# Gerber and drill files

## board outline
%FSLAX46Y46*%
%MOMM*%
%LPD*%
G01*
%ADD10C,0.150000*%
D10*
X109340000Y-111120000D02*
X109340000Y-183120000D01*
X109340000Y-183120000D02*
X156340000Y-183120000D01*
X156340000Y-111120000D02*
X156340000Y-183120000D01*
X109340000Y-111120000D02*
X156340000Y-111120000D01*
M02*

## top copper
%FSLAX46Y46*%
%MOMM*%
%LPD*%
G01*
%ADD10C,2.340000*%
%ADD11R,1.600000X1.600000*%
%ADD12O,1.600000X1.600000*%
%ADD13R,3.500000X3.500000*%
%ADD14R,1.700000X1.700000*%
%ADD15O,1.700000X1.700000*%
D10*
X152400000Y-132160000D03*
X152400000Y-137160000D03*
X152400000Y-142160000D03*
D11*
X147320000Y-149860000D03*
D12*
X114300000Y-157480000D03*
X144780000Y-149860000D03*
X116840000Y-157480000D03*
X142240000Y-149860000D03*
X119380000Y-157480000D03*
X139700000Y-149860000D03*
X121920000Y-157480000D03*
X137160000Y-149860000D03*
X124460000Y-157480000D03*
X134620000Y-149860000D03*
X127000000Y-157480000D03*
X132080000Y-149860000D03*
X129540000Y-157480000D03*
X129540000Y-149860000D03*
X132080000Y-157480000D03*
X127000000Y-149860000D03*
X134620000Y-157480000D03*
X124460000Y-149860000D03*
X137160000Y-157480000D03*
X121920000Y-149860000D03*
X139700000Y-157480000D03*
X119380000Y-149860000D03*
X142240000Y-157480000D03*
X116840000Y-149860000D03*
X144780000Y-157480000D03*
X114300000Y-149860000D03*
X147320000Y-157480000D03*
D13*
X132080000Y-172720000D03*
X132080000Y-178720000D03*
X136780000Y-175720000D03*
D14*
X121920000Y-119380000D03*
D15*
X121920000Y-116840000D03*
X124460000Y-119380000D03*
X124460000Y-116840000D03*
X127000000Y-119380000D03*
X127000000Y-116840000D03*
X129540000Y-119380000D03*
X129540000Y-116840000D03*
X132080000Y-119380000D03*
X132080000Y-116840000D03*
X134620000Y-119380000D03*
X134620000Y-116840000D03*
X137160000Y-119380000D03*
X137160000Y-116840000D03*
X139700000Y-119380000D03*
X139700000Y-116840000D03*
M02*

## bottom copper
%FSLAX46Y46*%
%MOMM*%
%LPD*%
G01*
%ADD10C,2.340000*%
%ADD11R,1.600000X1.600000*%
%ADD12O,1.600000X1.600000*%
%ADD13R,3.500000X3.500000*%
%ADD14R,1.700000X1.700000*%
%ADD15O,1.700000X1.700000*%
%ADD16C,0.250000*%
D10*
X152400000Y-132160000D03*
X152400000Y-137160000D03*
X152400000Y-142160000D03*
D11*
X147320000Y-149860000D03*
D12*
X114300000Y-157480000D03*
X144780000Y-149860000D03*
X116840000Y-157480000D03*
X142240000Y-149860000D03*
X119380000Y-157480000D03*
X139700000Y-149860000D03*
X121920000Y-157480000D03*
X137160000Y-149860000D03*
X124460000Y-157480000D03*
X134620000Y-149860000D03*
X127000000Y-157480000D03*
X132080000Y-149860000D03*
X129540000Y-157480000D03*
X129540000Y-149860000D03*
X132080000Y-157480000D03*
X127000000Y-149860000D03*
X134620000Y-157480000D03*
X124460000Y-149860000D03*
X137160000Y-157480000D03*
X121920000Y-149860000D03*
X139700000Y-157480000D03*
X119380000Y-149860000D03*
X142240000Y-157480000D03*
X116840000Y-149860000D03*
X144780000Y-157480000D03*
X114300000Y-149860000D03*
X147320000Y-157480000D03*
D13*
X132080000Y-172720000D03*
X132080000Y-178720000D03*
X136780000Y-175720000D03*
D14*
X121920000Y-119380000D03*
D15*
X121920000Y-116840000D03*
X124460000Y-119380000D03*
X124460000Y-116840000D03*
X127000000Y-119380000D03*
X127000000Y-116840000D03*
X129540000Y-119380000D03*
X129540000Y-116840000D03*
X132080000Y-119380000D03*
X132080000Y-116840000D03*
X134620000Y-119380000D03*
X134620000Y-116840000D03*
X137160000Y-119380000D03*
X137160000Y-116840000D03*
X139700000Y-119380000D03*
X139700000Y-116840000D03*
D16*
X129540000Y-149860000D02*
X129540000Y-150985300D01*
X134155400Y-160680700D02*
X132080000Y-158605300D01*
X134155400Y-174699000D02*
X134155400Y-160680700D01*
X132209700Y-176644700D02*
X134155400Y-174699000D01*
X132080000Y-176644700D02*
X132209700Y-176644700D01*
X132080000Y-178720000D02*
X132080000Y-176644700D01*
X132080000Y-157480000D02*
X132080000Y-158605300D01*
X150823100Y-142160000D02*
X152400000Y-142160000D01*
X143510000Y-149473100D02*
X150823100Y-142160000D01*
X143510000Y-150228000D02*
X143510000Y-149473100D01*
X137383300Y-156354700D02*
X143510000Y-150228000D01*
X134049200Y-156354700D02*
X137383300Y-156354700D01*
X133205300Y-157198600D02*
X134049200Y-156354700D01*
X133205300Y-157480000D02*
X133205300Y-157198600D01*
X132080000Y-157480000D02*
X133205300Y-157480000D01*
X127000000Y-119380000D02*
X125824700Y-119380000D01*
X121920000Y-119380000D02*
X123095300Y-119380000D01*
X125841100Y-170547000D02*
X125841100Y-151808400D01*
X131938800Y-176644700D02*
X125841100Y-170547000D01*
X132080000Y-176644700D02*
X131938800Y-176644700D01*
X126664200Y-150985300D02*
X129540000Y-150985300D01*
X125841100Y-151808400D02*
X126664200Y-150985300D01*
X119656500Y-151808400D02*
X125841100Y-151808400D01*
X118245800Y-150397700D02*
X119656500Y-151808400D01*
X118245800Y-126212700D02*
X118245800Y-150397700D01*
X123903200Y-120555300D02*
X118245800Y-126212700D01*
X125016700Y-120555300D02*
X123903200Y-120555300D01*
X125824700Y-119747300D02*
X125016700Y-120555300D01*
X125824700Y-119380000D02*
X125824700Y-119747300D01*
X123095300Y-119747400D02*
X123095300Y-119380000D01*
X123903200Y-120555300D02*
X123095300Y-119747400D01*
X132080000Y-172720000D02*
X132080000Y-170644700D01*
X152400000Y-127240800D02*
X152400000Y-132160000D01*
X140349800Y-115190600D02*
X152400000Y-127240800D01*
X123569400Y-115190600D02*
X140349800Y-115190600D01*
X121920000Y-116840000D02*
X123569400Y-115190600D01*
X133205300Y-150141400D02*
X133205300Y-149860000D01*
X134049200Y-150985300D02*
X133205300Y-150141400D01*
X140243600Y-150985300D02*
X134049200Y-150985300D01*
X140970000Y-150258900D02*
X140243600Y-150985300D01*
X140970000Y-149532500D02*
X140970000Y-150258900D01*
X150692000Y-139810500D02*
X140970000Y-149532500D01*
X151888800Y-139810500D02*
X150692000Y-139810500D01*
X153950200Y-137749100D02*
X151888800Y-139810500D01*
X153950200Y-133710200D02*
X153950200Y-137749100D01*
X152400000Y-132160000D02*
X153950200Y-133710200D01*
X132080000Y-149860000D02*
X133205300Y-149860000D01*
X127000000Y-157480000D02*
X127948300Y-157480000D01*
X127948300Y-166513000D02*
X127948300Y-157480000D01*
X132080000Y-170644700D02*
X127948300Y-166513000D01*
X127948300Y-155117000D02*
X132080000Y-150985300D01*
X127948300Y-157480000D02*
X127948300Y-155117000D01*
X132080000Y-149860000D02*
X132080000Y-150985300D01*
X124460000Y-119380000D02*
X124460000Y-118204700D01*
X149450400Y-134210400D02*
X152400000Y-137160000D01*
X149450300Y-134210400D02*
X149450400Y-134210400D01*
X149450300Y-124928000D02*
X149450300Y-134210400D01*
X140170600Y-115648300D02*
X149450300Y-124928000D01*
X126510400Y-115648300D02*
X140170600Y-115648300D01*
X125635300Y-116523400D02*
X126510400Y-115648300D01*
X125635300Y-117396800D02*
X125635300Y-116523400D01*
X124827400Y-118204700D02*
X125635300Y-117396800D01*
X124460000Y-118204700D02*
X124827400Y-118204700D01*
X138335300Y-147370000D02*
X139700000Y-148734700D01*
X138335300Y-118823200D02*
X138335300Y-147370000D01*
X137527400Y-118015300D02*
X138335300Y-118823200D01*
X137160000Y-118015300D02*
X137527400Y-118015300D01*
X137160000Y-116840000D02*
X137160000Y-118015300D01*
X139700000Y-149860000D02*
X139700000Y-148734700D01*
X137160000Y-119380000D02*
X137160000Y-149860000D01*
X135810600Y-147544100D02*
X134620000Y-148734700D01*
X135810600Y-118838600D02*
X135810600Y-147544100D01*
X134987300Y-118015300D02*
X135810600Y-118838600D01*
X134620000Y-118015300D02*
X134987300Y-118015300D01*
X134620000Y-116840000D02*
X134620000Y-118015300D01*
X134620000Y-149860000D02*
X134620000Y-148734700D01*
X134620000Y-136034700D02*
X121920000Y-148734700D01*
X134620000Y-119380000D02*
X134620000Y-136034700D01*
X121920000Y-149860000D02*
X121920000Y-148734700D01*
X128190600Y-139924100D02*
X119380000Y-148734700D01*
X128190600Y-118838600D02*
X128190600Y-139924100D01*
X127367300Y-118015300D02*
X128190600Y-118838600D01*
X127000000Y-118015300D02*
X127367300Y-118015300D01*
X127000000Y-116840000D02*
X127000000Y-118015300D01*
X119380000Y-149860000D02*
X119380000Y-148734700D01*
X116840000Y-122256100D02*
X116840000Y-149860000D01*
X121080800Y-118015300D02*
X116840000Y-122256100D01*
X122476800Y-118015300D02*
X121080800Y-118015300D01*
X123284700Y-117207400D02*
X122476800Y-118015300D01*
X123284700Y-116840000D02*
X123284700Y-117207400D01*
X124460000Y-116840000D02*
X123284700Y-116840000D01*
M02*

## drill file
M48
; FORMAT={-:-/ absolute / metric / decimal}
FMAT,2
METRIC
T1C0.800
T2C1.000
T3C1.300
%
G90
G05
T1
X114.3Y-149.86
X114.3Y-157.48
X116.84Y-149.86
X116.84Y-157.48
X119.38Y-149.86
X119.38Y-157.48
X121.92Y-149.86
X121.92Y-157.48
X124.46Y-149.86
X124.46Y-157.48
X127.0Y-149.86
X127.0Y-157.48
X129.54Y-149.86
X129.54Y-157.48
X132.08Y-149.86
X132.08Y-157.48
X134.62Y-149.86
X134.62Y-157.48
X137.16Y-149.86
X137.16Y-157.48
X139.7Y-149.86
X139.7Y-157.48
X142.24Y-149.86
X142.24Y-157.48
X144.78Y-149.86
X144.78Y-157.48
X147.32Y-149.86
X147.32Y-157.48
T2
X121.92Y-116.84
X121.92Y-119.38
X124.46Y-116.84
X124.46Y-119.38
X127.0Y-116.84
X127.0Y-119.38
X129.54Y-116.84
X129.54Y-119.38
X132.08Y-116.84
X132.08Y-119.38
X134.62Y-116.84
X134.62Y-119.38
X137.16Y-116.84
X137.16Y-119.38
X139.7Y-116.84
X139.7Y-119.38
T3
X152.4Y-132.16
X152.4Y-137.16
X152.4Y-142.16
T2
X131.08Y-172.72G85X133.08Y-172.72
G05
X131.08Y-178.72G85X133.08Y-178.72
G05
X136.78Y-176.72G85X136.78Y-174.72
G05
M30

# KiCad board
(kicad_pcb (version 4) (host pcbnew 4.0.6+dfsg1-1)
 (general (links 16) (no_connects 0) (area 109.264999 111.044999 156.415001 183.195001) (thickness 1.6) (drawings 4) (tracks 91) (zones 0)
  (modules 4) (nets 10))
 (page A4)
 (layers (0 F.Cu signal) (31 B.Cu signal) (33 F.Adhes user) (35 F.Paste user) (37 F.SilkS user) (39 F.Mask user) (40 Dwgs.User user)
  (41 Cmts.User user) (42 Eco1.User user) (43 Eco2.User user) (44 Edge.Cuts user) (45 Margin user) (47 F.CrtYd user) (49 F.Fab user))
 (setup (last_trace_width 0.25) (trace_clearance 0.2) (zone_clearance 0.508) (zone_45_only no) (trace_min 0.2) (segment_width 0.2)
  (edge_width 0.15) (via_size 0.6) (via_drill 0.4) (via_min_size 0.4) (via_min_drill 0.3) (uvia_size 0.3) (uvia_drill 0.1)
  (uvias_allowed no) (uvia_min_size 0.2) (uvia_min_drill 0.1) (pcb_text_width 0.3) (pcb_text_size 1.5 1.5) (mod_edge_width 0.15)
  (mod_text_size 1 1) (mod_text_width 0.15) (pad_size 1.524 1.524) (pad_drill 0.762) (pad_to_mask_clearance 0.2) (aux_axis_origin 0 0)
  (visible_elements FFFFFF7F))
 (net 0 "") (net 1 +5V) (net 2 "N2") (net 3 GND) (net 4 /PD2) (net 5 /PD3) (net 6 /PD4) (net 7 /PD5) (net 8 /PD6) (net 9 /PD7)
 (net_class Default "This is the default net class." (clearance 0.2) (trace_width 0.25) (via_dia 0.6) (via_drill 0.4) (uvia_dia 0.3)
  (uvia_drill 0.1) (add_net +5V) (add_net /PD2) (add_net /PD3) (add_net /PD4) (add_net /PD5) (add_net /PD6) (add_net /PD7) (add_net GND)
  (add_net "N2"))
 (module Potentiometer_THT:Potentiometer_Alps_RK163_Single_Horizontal (layer F.Cu) (at 152.4 142.16)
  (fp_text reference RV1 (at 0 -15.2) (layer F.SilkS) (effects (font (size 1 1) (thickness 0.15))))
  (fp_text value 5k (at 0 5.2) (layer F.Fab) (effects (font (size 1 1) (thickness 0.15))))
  (pad 3 thru_hole circle (at 0 -10) (size 2.34 2.34) (drill 1.3) (layers *.Cu *.Mask) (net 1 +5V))
  (pad 2 thru_hole circle (at 0 -5) (size 2.34 2.34) (drill 1.3) (layers *.Cu *.Mask) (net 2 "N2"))
  (pad 1 thru_hole circle (at 0 0) (size 2.34 2.34) (drill 1.3) (layers *.Cu *.Mask) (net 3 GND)))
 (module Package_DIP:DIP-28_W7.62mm (layer F.Cu) (at 147.32 149.86 270)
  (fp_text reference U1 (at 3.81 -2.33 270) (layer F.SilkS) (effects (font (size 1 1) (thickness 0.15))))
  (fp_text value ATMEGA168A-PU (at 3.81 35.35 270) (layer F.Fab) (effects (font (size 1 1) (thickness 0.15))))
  (pad 1 thru_hole rect (at 0 0 270) (size 1.6 1.6) (drill 0.8) (layers *.Cu *.Mask))
  (pad 15 thru_hole oval (at 7.62 33.02 270) (size 1.6 1.6) (drill 0.8) (layers *.Cu *.Mask))
  (pad 2 thru_hole oval (at 0 2.54 270) (size 1.6 1.6) (drill 0.8) (layers *.Cu *.Mask))
  (pad 16 thru_hole oval (at 7.62 30.48 270) (size 1.6 1.6) (drill 0.8) (layers *.Cu *.Mask))
  (pad 3 thru_hole oval (at 0 5.08 270) (size 1.6 1.6) (drill 0.8) (layers *.Cu *.Mask))
  (pad 17 thru_hole oval (at 7.62 27.94 270) (size 1.6 1.6) (drill 0.8) (layers *.Cu *.Mask))
  (pad 4 thru_hole oval (at 0 7.62 270) (size 1.6 1.6) (drill 0.8) (layers *.Cu *.Mask) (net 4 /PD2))
  (pad 18 thru_hole oval (at 7.62 25.4 270) (size 1.6 1.6) (drill 0.8) (layers *.Cu *.Mask))
  (pad 5 thru_hole oval (at 0 10.16 270) (size 1.6 1.6) (drill 0.8) (layers *.Cu *.Mask) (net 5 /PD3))
  (pad 19 thru_hole oval (at 7.62 22.86 270) (size 1.6 1.6) (drill 0.8) (layers *.Cu *.Mask))
  (pad 6 thru_hole oval (at 0 12.7 270) (size 1.6 1.6) (drill 0.8) (layers *.Cu *.Mask) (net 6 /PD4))
  (pad 20 thru_hole oval (at 7.62 20.32 270) (size 1.6 1.6) (drill 0.8) (layers *.Cu *.Mask) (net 1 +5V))
  (pad 7 thru_hole oval (at 0 15.24 270) (size 1.6 1.6) (drill 0.8) (layers *.Cu *.Mask) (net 1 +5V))
  (pad 21 thru_hole oval (at 7.62 17.78 270) (size 1.6 1.6) (drill 0.8) (layers *.Cu *.Mask))
  (pad 8 thru_hole oval (at 0 17.78 270) (size 1.6 1.6) (drill 0.8) (layers *.Cu *.Mask) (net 3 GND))
  (pad 22 thru_hole oval (at 7.62 15.24 270) (size 1.6 1.6) (drill 0.8) (layers *.Cu *.Mask) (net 3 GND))
  (pad 9 thru_hole oval (at 0 20.32 270) (size 1.6 1.6) (drill 0.8) (layers *.Cu *.Mask))
  (pad 23 thru_hole oval (at 7.62 12.7 270) (size 1.6 1.6) (drill 0.8) (layers *.Cu *.Mask))
  (pad 10 thru_hole oval (at 0 22.86 270) (size 1.6 1.6) (drill 0.8) (layers *.Cu *.Mask))
  (pad 24 thru_hole oval (at 7.62 10.16 270) (size 1.6 1.6) (drill 0.8) (layers *.Cu *.Mask))
  (pad 11 thru_hole oval (at 0 25.4 270) (size 1.6 1.6) (drill 0.8) (layers *.Cu *.Mask) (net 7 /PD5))
  (pad 25 thru_hole oval (at 7.62 7.62 270) (size 1.6 1.6) (drill 0.8) (layers *.Cu *.Mask))
  (pad 12 thru_hole oval (at 0 27.94 270) (size 1.6 1.6) (drill 0.8) (layers *.Cu *.Mask) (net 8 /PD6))
  (pad 26 thru_hole oval (at 7.62 5.08 270) (size 1.6 1.6) (drill 0.8) (layers *.Cu *.Mask))
  (pad 13 thru_hole oval (at 0 30.48 270) (size 1.6 1.6) (drill 0.8) (layers *.Cu *.Mask) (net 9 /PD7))
  (pad 27 thru_hole oval (at 7.62 2.54 270) (size 1.6 1.6) (drill 0.8) (layers *.Cu *.Mask))
  (pad 14 thru_hole oval (at 0 33.02 270) (size 1.6 1.6) (drill 0.8) (layers *.Cu *.Mask))
  (pad 28 thru_hole oval (at 7.62 0 270) (size 1.6 1.6) (drill 0.8) (layers *.Cu *.Mask)))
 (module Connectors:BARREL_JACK (layer F.Cu) (at 132.08 172.72 90)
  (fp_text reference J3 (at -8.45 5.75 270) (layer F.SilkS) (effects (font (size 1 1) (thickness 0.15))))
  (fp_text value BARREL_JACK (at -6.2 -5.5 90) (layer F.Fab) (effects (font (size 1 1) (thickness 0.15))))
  (pad 1 thru_hole rect (at 0 0 90) (size 3.5 3.5) (drill oval 1 3) (layers *.Cu *.Mask) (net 1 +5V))
  (pad 2 thru_hole rect (at -6 0 90) (size 3.5 3.5) (drill oval 1 3) (layers *.Cu *.Mask) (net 3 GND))
  (pad 3 thru_hole rect (at -3 4.7 90) (size 3.5 3.5) (drill oval 3 1) (layers *.Cu *.Mask)))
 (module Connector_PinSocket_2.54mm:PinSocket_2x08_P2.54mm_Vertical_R (layer F.Cu) (at 139.7 119.38 270)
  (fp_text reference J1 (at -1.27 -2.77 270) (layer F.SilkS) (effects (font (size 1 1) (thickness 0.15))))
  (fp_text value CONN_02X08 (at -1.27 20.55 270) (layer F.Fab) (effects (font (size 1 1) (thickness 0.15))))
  (pad 1 thru_hole rect (at 0 17.78 270) (size 1.7 1.7) (drill 1) (layers *.Cu *.Mask) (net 3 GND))
  (pad 2 thru_hole oval (at -2.54 17.78 270) (size 1.7 1.7) (drill 1) (layers *.Cu *.Mask) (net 1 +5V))
  (pad 3 thru_hole oval (at 0 15.24 270) (size 1.7 1.7) (drill 1) (layers *.Cu *.Mask) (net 2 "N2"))
  (pad 4 thru_hole oval (at -2.54 15.24 270) (size 1.7 1.7) (drill 1) (layers *.Cu *.Mask) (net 9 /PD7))
  (pad 5 thru_hole oval (at 0 12.7 270) (size 1.7 1.7) (drill 1) (layers *.Cu *.Mask) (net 3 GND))
  (pad 6 thru_hole oval (at -2.54 12.7 270) (size 1.7 1.7) (drill 1) (layers *.Cu *.Mask) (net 8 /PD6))
  (pad 7 thru_hole oval (at 0 10.16 270) (size 1.7 1.7) (drill 1) (layers *.Cu *.Mask))
  (pad 8 thru_hole oval (at -2.54 10.16 270) (size 1.7 1.7) (drill 1) (layers *.Cu *.Mask))
  (pad 9 thru_hole oval (at 0 7.62 270) (size 1.7 1.7) (drill 1) (layers *.Cu *.Mask))
  (pad 10 thru_hole oval (at -2.54 7.62 270) (size 1.7 1.7) (drill 1) (layers *.Cu *.Mask))
  (pad 11 thru_hole oval (at 0 5.08 270) (size 1.7 1.7) (drill 1) (layers *.Cu *.Mask) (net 7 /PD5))
  (pad 12 thru_hole oval (at -2.54 5.08 270) (size 1.7 1.7) (drill 1) (layers *.Cu *.Mask) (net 6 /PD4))
  (pad 13 thru_hole oval (at 0 2.54 270) (size 1.7 1.7) (drill 1) (layers *.Cu *.Mask) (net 5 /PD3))
  (pad 14 thru_hole oval (at -2.54 2.54 270) (size 1.7 1.7) (drill 1) (layers *.Cu *.Mask) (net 4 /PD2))
  (pad 15 thru_hole oval (at 0 0 270) (size 1.7 1.7) (drill 1) (layers *.Cu *.Mask))
  (pad 16 thru_hole oval (at -2.54 0 270) (size 1.7 1.7) (drill 1) (layers *.Cu *.Mask)))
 (gr_line (start 109.34 111.12) (end 109.34 183.12) (layer Edge.Cuts) (width 0.15))
 (gr_line (start 109.34 183.12) (end 156.34 183.12) (layer Edge.Cuts) (width 0.15))
 (gr_line (start 156.34 111.12) (end 156.34 183.12) (layer Edge.Cuts) (width 0.15))
 (gr_line (start 109.34 111.12) (end 156.34 111.12) (layer Edge.Cuts) (width 0.15))
 (segment (start 129.54 149.86) (end 129.54 150.9853) (width 0.25) (layer B.Cu) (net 3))
 (segment (start 134.1554 160.6807) (end 132.08 158.6053) (width 0.25) (layer B.Cu) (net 3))
 (segment (start 134.1554 174.699) (end 134.1554 160.6807) (width 0.25) (layer B.Cu) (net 3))
 (segment (start 132.2097 176.6447) (end 134.1554 174.699) (width 0.25) (layer B.Cu) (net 3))
 (segment (start 132.08 176.6447) (end 132.2097 176.6447) (width 0.25) (layer B.Cu) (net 3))
 (segment (start 132.08 178.72) (end 132.08 176.6447) (width 0.25) (layer B.Cu) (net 3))
 (segment (start 132.08 157.48) (end 132.08 158.6053) (width 0.25) (layer B.Cu) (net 3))
 (segment (start 150.8231 142.16) (end 152.4 142.16) (width 0.25) (layer B.Cu) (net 3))
 (segment (start 143.51 149.4731) (end 150.8231 142.16) (width 0.25) (layer B.Cu) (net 3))
 (segment (start 143.51 150.228) (end 143.51 149.4731) (width 0.25) (layer B.Cu) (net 3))
 (segment (start 137.3833 156.3547) (end 143.51 150.228) (width 0.25) (layer B.Cu) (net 3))
 (segment (start 134.0492 156.3547) (end 137.3833 156.3547) (width 0.25) (layer B.Cu) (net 3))
 (segment (start 133.2053 157.1986) (end 134.0492 156.3547) (width 0.25) (layer B.Cu) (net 3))
 (segment (start 133.2053 157.48) (end 133.2053 157.1986) (width 0.25) (layer B.Cu) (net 3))
 (segment (start 132.08 157.48) (end 133.2053 157.48) (width 0.25) (layer B.Cu) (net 3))
 (segment (start 127 119.38) (end 125.8247 119.38) (width 0.25) (layer B.Cu) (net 3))
 (segment (start 121.92 119.38) (end 123.0953 119.38) (width 0.25) (layer B.Cu) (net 3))
 (segment (start 125.8411 170.547) (end 125.8411 151.8084) (width 0.25) (layer B.Cu) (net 3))
 (segment (start 131.9388 176.6447) (end 125.8411 170.547) (width 0.25) (layer B.Cu) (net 3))
 (segment (start 132.08 176.6447) (end 131.9388 176.6447) (width 0.25) (layer B.Cu) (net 3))
 (segment (start 126.6642 150.9853) (end 129.54 150.9853) (width 0.25) (layer B.Cu) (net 3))
 (segment (start 125.8411 151.8084) (end 126.6642 150.9853) (width 0.25) (layer B.Cu) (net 3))
 (segment (start 119.6565 151.8084) (end 125.8411 151.8084) (width 0.25) (layer B.Cu) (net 3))
 (segment (start 118.2458 150.3977) (end 119.6565 151.8084) (width 0.25) (layer B.Cu) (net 3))
 (segment (start 118.2458 126.2127) (end 118.2458 150.3977) (width 0.25) (layer B.Cu) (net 3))
 (segment (start 123.9032 120.5553) (end 118.2458 126.2127) (width 0.25) (layer B.Cu) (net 3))
 (segment (start 125.0167 120.5553) (end 123.9032 120.5553) (width 0.25) (layer B.Cu) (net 3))
 (segment (start 125.8247 119.7473) (end 125.0167 120.5553) (width 0.25) (layer B.Cu) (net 3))
 (segment (start 125.8247 119.38) (end 125.8247 119.7473) (width 0.25) (layer B.Cu) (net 3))
 (segment (start 123.0953 119.7474) (end 123.0953 119.38) (width 0.25) (layer B.Cu) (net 3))
 (segment (start 123.9032 120.5553) (end 123.0953 119.7474) (width 0.25) (layer B.Cu) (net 3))
 (segment (start 132.08 172.72) (end 132.08 170.6447) (width 0.25) (layer B.Cu) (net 1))
 (segment (start 152.4 127.2408) (end 152.4 132.16) (width 0.25) (layer B.Cu) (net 1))
 (segment (start 140.3498 115.1906) (end 152.4 127.2408) (width 0.25) (layer B.Cu) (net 1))
 (segment (start 123.5694 115.1906) (end 140.3498 115.1906) (width 0.25) (layer B.Cu) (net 1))
 (segment (start 121.92 116.84) (end 123.5694 115.1906) (width 0.25) (layer B.Cu) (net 1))
 (segment (start 133.2053 150.1414) (end 133.2053 149.86) (width 0.25) (layer B.Cu) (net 1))
 (segment (start 134.0492 150.9853) (end 133.2053 150.1414) (width 0.25) (layer B.Cu) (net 1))
 (segment (start 140.2436 150.9853) (end 134.0492 150.9853) (width 0.25) (layer B.Cu) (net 1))
 (segment (start 140.97 150.2589) (end 140.2436 150.9853) (width 0.25) (layer B.Cu) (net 1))
 (segment (start 140.97 149.5325) (end 140.97 150.2589) (width 0.25) (layer B.Cu) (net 1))
 (segment (start 150.692 139.8105) (end 140.97 149.5325) (width 0.25) (layer B.Cu) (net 1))
 (segment (start 151.8888 139.8105) (end 150.692 139.8105) (width 0.25) (layer B.Cu) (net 1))
 (segment (start 153.9502 137.7491) (end 151.8888 139.8105) (width 0.25) (layer B.Cu) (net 1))
 (segment (start 153.9502 133.7102) (end 153.9502 137.7491) (width 0.25) (layer B.Cu) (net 1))
 (segment (start 152.4 132.16) (end 153.9502 133.7102) (width 0.25) (layer B.Cu) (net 1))
 (segment (start 132.08 149.86) (end 133.2053 149.86) (width 0.25) (layer B.Cu) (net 1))
 (segment (start 127 157.48) (end 127.9483 157.48) (width 0.25) (layer B.Cu) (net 1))
 (segment (start 127.9483 166.513) (end 127.9483 157.48) (width 0.25) (layer B.Cu) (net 1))
 (segment (start 132.08 170.6447) (end 127.9483 166.513) (width 0.25) (layer B.Cu) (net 1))
 (segment (start 127.9483 155.117) (end 132.08 150.9853) (width 0.25) (layer B.Cu) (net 1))
 (segment (start 127.9483 157.48) (end 127.9483 155.117) (width 0.25) (layer B.Cu) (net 1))
 (segment (start 132.08 149.86) (end 132.08 150.9853) (width 0.25) (layer B.Cu) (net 1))
 (segment (start 124.46 119.38) (end 124.46 118.2047) (width 0.25) (layer B.Cu) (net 2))
 (segment (start 149.4504 134.2104) (end 152.4 137.16) (width 0.25) (layer B.Cu) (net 2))
 (segment (start 149.4503 134.2104) (end 149.4504 134.2104) (width 0.25) (layer B.Cu) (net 2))
 (segment (start 149.4503 124.928) (end 149.4503 134.2104) (width 0.25) (layer B.Cu) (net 2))
 (segment (start 140.1706 115.6483) (end 149.4503 124.928) (width 0.25) (layer B.Cu) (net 2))
 (segment (start 126.5104 115.6483) (end 140.1706 115.6483) (width 0.25) (layer B.Cu) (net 2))
 (segment (start 125.6353 116.5234) (end 126.5104 115.6483) (width 0.25) (layer B.Cu) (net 2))
 (segment (start 125.6353 117.3968) (end 125.6353 116.5234) (width 0.25) (layer B.Cu) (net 2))
 (segment (start 124.8274 118.2047) (end 125.6353 117.3968) (width 0.25) (layer B.Cu) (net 2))
 (segment (start 124.46 118.2047) (end 124.8274 118.2047) (width 0.25) (layer B.Cu) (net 2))
 (segment (start 138.3353 147.37) (end 139.7 148.7347) (width 0.25) (layer B.Cu) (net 4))
 (segment (start 138.3353 118.8232) (end 138.3353 147.37) (width 0.25) (layer B.Cu) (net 4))
 (segment (start 137.5274 118.0153) (end 138.3353 118.8232) (width 0.25) (layer B.Cu) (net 4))
 (segment (start 137.16 118.0153) (end 137.5274 118.0153) (width 0.25) (layer B.Cu) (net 4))
 (segment (start 137.16 116.84) (end 137.16 118.0153) (width 0.25) (layer B.Cu) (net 4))
 (segment (start 139.7 149.86) (end 139.7 148.7347) (width 0.25) (layer B.Cu) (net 4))
 (segment (start 137.16 119.38) (end 137.16 149.86) (width 0.25) (layer B.Cu) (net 5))
 (segment (start 135.8106 147.5441) (end 134.62 148.7347) (width 0.25) (layer B.Cu) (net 6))
 (segment (start 135.8106 118.8386) (end 135.8106 147.5441) (width 0.25) (layer B.Cu) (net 6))
 (segment (start 134.9873 118.0153) (end 135.8106 118.8386) (width 0.25) (layer B.Cu) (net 6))
 (segment (start 134.62 118.0153) (end 134.9873 118.0153) (width 0.25) (layer B.Cu) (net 6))
 (segment (start 134.62 116.84) (end 134.62 118.0153) (width 0.25) (layer B.Cu) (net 6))
 (segment (start 134.62 149.86) (end 134.62 148.7347) (width 0.25) (layer B.Cu) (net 6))
 (segment (start 134.62 136.0347) (end 121.92 148.7347) (width 0.25) (layer B.Cu) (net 7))
 (segment (start 134.62 119.38) (end 134.62 136.0347) (width 0.25) (layer B.Cu) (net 7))
 (segment (start 121.92 149.86) (end 121.92 148.7347) (width 0.25) (layer B.Cu) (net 7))
 (segment (start 128.1906 139.9241) (end 119.38 148.7347) (width 0.25) (layer B.Cu) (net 8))
 (segment (start 128.1906 118.8386) (end 128.1906 139.9241) (width 0.25) (layer B.Cu) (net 8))
 (segment (start 127.3673 118.0153) (end 128.1906 118.8386) (width 0.25) (layer B.Cu) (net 8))
 (segment (start 127 118.0153) (end 127.3673 118.0153) (width 0.25) (layer B.Cu) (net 8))
 (segment (start 127 116.84) (end 127 118.0153) (width 0.25) (layer B.Cu) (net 8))
 (segment (start 119.38 149.86) (end 119.38 148.7347) (width 0.25) (layer B.Cu) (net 8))
 (segment (start 116.84 122.2561) (end 116.84 149.86) (width 0.25) (layer B.Cu) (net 9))
 (segment (start 121.0808 118.0153) (end 116.84 122.2561) (width 0.25) (layer B.Cu) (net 9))
 (segment (start 122.4768 118.0153) (end 121.0808 118.0153) (width 0.25) (layer B.Cu) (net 9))
 (segment (start 123.2847 117.2074) (end 122.4768 118.0153) (width 0.25) (layer B.Cu) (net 9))
 (segment (start 123.2847 116.84) (end 123.2847 117.2074) (width 0.25) (layer B.Cu) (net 9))
 (segment (start 124.46 116.84) (end 123.2847 116.84) (width 0.25) (layer B.Cu) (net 9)))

